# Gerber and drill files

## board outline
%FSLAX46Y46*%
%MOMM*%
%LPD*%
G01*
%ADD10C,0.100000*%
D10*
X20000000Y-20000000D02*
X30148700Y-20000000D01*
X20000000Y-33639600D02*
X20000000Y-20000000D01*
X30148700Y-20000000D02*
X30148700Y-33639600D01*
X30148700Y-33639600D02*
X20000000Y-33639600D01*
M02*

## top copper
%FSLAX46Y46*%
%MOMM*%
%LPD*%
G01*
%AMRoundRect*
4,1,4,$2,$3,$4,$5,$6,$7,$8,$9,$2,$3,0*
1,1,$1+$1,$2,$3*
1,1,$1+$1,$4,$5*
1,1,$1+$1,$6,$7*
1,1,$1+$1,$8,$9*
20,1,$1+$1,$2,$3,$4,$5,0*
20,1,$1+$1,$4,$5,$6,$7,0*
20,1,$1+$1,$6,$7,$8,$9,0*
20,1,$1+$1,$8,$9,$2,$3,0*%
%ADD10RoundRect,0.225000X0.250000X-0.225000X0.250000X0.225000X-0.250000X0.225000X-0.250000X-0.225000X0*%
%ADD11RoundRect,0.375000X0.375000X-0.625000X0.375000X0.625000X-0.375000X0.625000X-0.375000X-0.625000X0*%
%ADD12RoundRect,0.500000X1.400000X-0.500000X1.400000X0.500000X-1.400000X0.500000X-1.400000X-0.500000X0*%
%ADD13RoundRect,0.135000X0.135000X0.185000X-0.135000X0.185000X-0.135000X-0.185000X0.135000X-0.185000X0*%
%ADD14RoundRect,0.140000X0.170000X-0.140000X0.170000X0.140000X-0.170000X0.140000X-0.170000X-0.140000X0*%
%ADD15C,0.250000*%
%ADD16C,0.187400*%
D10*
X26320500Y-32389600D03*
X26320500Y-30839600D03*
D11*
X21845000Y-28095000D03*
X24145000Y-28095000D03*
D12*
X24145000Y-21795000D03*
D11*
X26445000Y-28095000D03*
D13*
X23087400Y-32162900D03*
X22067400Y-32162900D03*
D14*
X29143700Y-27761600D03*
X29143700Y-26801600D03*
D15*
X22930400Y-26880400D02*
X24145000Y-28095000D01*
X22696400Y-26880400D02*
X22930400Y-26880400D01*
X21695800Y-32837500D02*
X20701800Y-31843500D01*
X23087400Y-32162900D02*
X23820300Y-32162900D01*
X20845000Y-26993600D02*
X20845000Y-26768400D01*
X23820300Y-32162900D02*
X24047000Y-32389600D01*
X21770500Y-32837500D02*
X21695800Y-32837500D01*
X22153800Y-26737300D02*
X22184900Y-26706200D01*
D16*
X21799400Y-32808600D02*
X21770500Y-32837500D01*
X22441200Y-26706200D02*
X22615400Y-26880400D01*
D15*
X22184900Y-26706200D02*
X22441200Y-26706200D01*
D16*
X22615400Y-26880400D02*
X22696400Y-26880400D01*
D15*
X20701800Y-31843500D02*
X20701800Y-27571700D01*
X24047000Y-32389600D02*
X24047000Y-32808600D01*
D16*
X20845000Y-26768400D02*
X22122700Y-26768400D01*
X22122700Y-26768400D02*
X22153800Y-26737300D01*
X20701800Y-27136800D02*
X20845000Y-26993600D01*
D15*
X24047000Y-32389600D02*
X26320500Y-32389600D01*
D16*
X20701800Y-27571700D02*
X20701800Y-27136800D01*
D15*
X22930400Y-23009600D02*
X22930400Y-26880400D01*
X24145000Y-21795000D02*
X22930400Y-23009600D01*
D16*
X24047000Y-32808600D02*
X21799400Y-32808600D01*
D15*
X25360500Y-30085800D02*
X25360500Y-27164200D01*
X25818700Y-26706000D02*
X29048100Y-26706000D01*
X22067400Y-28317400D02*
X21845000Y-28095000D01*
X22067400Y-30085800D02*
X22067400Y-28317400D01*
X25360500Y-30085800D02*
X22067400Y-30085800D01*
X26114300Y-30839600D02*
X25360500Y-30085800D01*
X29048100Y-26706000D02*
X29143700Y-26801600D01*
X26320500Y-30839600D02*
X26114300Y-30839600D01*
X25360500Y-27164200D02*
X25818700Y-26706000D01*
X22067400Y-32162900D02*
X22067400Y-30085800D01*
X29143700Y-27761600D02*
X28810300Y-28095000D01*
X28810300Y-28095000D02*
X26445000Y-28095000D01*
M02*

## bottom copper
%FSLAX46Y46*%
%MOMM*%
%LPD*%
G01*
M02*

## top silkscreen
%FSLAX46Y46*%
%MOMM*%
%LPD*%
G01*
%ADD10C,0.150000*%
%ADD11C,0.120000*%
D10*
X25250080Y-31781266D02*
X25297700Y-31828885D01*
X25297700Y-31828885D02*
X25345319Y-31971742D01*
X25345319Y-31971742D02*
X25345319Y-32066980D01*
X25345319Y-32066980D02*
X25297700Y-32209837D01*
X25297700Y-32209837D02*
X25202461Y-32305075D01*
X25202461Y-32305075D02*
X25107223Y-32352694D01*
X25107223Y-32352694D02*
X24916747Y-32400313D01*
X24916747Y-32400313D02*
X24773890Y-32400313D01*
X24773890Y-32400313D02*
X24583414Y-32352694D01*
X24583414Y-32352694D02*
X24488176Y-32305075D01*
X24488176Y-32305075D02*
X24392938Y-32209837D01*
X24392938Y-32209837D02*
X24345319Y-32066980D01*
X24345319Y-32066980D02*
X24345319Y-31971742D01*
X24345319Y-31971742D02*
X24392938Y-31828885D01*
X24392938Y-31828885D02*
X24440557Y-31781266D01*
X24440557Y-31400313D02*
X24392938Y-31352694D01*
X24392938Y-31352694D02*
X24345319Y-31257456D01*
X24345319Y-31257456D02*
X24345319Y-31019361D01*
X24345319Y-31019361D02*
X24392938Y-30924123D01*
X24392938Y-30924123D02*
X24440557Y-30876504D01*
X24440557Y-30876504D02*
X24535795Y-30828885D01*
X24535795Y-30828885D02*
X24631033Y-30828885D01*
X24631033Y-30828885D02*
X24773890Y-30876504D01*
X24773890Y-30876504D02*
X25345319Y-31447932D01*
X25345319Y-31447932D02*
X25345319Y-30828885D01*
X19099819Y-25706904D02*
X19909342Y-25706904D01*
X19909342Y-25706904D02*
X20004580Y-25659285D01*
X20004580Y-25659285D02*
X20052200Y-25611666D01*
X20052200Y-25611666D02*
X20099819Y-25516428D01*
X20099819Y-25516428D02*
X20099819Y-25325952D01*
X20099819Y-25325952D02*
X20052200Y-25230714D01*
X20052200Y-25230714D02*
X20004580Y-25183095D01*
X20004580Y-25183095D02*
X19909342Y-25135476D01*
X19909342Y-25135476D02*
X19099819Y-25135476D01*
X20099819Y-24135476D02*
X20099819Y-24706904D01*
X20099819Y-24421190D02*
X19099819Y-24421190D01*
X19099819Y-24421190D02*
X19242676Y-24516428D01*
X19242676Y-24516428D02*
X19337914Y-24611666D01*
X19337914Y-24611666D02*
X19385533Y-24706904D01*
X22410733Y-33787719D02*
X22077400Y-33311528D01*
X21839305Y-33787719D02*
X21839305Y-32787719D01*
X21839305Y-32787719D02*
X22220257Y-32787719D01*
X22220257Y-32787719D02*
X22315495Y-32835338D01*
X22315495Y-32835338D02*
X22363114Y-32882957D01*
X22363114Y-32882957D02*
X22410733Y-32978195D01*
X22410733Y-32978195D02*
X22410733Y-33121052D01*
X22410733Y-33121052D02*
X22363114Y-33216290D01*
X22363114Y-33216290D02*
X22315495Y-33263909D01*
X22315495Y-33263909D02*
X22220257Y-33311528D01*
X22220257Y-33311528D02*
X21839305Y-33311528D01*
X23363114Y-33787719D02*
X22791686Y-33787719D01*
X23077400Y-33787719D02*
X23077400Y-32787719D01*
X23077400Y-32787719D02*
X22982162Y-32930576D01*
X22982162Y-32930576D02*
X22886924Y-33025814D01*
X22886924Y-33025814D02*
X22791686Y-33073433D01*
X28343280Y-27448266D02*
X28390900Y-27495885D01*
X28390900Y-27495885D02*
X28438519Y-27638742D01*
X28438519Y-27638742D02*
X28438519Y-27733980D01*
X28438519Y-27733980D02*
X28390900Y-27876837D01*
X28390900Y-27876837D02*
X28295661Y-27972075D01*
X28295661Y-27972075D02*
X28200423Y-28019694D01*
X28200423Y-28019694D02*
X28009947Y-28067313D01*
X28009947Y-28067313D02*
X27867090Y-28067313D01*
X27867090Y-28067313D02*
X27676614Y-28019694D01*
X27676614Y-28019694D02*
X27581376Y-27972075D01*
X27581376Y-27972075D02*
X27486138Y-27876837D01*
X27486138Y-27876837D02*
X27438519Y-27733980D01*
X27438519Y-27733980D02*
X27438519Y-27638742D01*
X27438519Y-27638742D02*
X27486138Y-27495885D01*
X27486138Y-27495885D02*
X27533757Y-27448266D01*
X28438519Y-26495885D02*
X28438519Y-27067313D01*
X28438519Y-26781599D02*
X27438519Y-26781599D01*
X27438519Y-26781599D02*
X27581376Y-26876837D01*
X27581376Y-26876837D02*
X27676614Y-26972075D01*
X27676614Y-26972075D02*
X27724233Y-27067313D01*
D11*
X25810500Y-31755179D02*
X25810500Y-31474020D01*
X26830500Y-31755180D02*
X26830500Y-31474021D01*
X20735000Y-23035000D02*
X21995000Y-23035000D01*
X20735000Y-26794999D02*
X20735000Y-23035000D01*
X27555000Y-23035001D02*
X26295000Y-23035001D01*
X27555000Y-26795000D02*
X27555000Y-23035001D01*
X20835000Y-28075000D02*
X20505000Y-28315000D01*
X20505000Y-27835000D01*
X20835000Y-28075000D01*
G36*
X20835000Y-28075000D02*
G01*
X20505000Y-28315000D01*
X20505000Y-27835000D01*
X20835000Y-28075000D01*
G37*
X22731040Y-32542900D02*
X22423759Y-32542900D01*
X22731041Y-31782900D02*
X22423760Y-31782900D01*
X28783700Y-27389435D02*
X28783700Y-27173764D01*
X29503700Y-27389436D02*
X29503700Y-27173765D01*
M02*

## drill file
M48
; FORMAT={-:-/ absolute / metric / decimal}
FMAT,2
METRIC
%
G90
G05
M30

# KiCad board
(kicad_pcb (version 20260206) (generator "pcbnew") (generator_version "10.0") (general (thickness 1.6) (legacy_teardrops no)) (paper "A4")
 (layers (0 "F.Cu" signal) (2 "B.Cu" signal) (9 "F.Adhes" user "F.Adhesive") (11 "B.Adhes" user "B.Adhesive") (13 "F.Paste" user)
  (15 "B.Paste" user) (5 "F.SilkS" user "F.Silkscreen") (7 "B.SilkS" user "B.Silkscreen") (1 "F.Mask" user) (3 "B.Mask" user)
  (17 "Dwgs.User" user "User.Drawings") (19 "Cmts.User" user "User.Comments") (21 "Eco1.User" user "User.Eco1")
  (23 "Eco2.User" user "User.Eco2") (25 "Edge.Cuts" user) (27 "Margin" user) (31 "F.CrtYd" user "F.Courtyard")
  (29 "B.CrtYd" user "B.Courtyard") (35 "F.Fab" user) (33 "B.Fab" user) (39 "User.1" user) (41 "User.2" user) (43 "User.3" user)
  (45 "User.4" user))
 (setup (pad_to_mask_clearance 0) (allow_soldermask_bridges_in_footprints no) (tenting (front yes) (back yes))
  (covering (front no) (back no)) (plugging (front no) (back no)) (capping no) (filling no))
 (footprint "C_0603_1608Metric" (layer "F.Cu") (at 26.3205 31.6146 90)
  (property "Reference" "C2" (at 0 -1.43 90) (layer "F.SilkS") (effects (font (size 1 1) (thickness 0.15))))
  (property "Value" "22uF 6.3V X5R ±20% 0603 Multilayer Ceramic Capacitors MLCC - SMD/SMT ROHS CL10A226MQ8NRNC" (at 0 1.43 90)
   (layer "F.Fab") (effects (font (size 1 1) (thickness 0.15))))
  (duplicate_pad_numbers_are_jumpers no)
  (fp_line (start -0.140579 -0.51) (end 0.14058 -0.51) (stroke (width 0.12) (type solid)) (layer "F.SilkS"))
  (fp_line (start -0.14058 0.51) (end 0.140579 0.51) (stroke (width 0.12) (type solid)) (layer "F.SilkS"))
  (pad "1" smd roundrect (at -0.775 0 90) (size 0.9 0.95) (layers "F.Cu" "F.Mask" "F.Paste") (roundrect_rratio 0.25) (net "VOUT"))
  (pad "2" smd roundrect (at 0.775 0 90) (size 0.9 0.95) (layers "F.Cu" "F.Mask" "F.Paste") (roundrect_rratio 0.25) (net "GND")))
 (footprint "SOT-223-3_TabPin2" (layer "F.Cu") (at 24.145 24.945 90)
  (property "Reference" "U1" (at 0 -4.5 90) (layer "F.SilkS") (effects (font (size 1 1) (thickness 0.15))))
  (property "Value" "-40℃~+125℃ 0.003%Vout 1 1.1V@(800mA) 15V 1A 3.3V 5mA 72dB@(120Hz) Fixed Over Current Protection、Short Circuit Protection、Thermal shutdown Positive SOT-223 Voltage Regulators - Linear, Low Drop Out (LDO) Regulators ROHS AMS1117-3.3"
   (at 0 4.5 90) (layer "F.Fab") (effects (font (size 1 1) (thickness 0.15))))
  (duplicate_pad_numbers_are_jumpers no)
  (fp_line (start 1.91 -3.41) (end 1.91 -2.15) (stroke (width 0.12) (type solid)) (layer "F.SilkS"))
  (fp_line (start -1.849999 -3.41) (end 1.91 -3.41) (stroke (width 0.12) (type solid)) (layer "F.SilkS"))
  (fp_line (start 1.909999 3.41) (end 1.909999 2.15) (stroke (width 0.12) (type solid)) (layer "F.SilkS"))
  (fp_line (start -1.85 3.41) (end 1.909999 3.41) (stroke (width 0.12) (type solid)) (layer "F.SilkS"))
  (fp_poly (pts (xy -3.13 -3.31) (xy -3.37 -3.64) (xy -2.89 -3.64)) (stroke (width 0.12) (type solid)) (fill yes) (layer "F.SilkS"))
  (pad "1" smd roundrect (at -3.15 -2.3 90) (size 2 1.5) (layers "F.Cu" "F.Mask" "F.Paste") (roundrect_rratio 0.25) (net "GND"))
  (pad "2" smd roundrect (at -3.15 0 90) (size 2 1.5) (layers "F.Cu" "F.Mask" "F.Paste") (roundrect_rratio 0.25) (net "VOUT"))
  (pad "2" smd roundrect (at 3.15 0 90) (size 2 3.8) (layers "F.Cu" "F.Mask" "F.Paste") (roundrect_rratio 0.25) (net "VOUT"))
  (pad "3" smd roundrect (at -3.15 2.3 90) (size 2 1.5) (layers "F.Cu" "F.Mask" "F.Paste") (roundrect_rratio 0.25) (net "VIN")))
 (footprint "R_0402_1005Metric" (layer "F.Cu") (at 22.5774 32.1629 180)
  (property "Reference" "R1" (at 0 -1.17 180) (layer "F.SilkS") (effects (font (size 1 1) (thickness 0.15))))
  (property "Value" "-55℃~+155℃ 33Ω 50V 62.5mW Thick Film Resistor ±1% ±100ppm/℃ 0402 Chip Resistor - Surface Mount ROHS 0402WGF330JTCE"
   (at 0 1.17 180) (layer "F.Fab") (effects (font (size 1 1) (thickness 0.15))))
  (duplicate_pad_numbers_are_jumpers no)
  (fp_line (start -0.15364 -0.38) (end 0.153641 -0.38) (stroke (width 0.12) (type solid)) (layer "F.SilkS"))
  (fp_line (start -0.153641 0.38) (end 0.15364 0.38) (stroke (width 0.12) (type solid)) (layer "F.SilkS"))
  (pad "1" smd roundrect (at -0.51 0 180) (size 0.54 0.64) (layers "F.Cu" "F.Mask" "F.Paste") (roundrect_rratio 0.25) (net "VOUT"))
  (pad "2" smd roundrect (at 0.51 0 180) (size 0.54 0.64) (layers "F.Cu" "F.Mask" "F.Paste") (roundrect_rratio 0.25) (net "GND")))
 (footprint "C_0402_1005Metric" (layer "F.Cu") (at 29.1437 27.2816 90)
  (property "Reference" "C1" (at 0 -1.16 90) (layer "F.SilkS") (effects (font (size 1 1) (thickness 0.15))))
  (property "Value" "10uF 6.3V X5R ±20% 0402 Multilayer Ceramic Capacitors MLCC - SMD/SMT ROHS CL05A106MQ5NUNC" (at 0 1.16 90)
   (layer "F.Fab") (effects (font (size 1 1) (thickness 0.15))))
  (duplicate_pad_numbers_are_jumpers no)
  (fp_line (start -0.107835 -0.36) (end 0.107836 -0.36) (stroke (width 0.12) (type solid)) (layer "F.SilkS"))
  (fp_line (start -0.107836 0.36) (end 0.107835 0.36) (stroke (width 0.12) (type solid)) (layer "F.SilkS"))
  (pad "1" smd roundrect (at -0.48 0 90) (size 0.56 0.62) (layers "F.Cu" "F.Mask" "F.Paste") (roundrect_rratio 0.25) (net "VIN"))
  (pad "2" smd roundrect (at 0.48 0 90) (size 0.56 0.62) (layers "F.Cu" "F.Mask" "F.Paste") (roundrect_rratio 0.25) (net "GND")))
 (gr_line (start 20 20) (end 30.1487 20) (stroke (width 0.1) (type default)) (layer "Edge.Cuts"))
 (gr_line (start 20 33.6396) (end 20 20) (stroke (width 0.1) (type default)) (layer "Edge.Cuts"))
 (gr_line (start 30.1487 20) (end 30.1487 33.6396) (stroke (width 0.1) (type default)) (layer "Edge.Cuts"))
 (gr_line (start 30.1487 33.6396) (end 20 33.6396) (stroke (width 0.1) (type default)) (layer "Edge.Cuts"))
 (segment (start 22.9304 26.8804) (end 24.145 28.095) (width 0.25) (layer "F.Cu") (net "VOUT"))
 (segment (start 22.6964 26.8804) (end 22.9304 26.8804) (width 0.25) (layer "F.Cu") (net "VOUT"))
 (segment (start 21.6958 32.8375) (end 20.7018 31.8435) (width 0.25) (layer "F.Cu") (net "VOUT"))
 (segment (start 23.0874 32.1629) (end 23.8203 32.1629) (width 0.25) (layer "F.Cu") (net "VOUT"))
 (segment (start 20.845 26.9936) (end 20.845 26.7684) (width 0.25) (layer "F.Cu") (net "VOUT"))
 (segment (start 23.8203 32.1629) (end 24.047 32.3896) (width 0.25) (layer "F.Cu") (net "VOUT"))
 (segment (start 21.7705 32.8375) (end 21.6958 32.8375) (width 0.25) (layer "F.Cu") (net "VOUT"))
 (segment (start 22.1538 26.7373) (end 22.1849 26.7062) (width 0.25) (layer "F.Cu") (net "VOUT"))
 (segment (start 21.7994 32.8086) (end 21.7705 32.8375) (width 0.1874) (layer "F.Cu") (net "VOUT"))
 (segment (start 22.4412 26.7062) (end 22.6154 26.8804) (width 0.1874) (layer "F.Cu") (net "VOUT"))
 (segment (start 22.1849 26.7062) (end 22.4412 26.7062) (width 0.25) (layer "F.Cu") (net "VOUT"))
 (segment (start 22.6154 26.8804) (end 22.6964 26.8804) (width 0.1874) (layer "F.Cu") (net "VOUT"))
 (segment (start 20.7018 31.8435) (end 20.7018 27.5717) (width 0.25) (layer "F.Cu") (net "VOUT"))
 (segment (start 24.047 32.3896) (end 24.047 32.8086) (width 0.25) (layer "F.Cu") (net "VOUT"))
 (segment (start 20.845 26.7684) (end 22.1227 26.7684) (width 0.1874) (layer "F.Cu") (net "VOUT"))
 (segment (start 22.1227 26.7684) (end 22.1538 26.7373) (width 0.1874) (layer "F.Cu") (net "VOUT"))
 (segment (start 20.7018 27.1368) (end 20.845 26.9936) (width 0.1874) (layer "F.Cu") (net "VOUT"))
 (segment (start 24.047 32.3896) (end 26.3205 32.3896) (width 0.25) (layer "F.Cu") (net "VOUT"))
 (segment (start 20.7018 27.5717) (end 20.7018 27.1368) (width 0.1874) (layer "F.Cu") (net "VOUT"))
 (segment (start 22.9304 23.0096) (end 22.9304 26.8804) (width 0.25) (layer "F.Cu") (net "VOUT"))
 (segment (start 24.145 21.795) (end 22.9304 23.0096) (width 0.25) (layer "F.Cu") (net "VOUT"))
 (segment (start 24.047 32.8086) (end 21.7994 32.8086) (width 0.1874) (layer "F.Cu") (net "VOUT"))
 (segment (start 25.3605 30.0858) (end 25.3605 27.1642) (width 0.25) (layer "F.Cu") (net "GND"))
 (segment (start 25.8187 26.706) (end 29.0481 26.706) (width 0.25) (layer "F.Cu") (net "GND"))
 (segment (start 22.0674 28.3174) (end 21.845 28.095) (width 0.25) (layer "F.Cu") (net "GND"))
 (segment (start 22.0674 30.0858) (end 22.0674 28.3174) (width 0.25) (layer "F.Cu") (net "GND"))
 (segment (start 25.3605 30.0858) (end 22.0674 30.0858) (width 0.25) (layer "F.Cu") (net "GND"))
 (segment (start 26.1143 30.8396) (end 25.3605 30.0858) (width 0.25) (layer "F.Cu") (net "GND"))
 (segment (start 29.0481 26.706) (end 29.1437 26.8016) (width 0.25) (layer "F.Cu") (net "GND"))
 (segment (start 26.3205 30.8396) (end 26.1143 30.8396) (width 0.25) (layer "F.Cu") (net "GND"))
 (segment (start 25.3605 27.1642) (end 25.8187 26.706) (width 0.25) (layer "F.Cu") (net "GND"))
 (segment (start 22.0674 32.1629) (end 22.0674 30.0858) (width 0.25) (layer "F.Cu") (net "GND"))
 (segment (start 29.1437 27.7616) (end 28.8103 28.095) (width 0.25) (layer "F.Cu") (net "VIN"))
 (segment (start 28.8103 28.095) (end 26.445 28.095) (width 0.25) (layer "F.Cu") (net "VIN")))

